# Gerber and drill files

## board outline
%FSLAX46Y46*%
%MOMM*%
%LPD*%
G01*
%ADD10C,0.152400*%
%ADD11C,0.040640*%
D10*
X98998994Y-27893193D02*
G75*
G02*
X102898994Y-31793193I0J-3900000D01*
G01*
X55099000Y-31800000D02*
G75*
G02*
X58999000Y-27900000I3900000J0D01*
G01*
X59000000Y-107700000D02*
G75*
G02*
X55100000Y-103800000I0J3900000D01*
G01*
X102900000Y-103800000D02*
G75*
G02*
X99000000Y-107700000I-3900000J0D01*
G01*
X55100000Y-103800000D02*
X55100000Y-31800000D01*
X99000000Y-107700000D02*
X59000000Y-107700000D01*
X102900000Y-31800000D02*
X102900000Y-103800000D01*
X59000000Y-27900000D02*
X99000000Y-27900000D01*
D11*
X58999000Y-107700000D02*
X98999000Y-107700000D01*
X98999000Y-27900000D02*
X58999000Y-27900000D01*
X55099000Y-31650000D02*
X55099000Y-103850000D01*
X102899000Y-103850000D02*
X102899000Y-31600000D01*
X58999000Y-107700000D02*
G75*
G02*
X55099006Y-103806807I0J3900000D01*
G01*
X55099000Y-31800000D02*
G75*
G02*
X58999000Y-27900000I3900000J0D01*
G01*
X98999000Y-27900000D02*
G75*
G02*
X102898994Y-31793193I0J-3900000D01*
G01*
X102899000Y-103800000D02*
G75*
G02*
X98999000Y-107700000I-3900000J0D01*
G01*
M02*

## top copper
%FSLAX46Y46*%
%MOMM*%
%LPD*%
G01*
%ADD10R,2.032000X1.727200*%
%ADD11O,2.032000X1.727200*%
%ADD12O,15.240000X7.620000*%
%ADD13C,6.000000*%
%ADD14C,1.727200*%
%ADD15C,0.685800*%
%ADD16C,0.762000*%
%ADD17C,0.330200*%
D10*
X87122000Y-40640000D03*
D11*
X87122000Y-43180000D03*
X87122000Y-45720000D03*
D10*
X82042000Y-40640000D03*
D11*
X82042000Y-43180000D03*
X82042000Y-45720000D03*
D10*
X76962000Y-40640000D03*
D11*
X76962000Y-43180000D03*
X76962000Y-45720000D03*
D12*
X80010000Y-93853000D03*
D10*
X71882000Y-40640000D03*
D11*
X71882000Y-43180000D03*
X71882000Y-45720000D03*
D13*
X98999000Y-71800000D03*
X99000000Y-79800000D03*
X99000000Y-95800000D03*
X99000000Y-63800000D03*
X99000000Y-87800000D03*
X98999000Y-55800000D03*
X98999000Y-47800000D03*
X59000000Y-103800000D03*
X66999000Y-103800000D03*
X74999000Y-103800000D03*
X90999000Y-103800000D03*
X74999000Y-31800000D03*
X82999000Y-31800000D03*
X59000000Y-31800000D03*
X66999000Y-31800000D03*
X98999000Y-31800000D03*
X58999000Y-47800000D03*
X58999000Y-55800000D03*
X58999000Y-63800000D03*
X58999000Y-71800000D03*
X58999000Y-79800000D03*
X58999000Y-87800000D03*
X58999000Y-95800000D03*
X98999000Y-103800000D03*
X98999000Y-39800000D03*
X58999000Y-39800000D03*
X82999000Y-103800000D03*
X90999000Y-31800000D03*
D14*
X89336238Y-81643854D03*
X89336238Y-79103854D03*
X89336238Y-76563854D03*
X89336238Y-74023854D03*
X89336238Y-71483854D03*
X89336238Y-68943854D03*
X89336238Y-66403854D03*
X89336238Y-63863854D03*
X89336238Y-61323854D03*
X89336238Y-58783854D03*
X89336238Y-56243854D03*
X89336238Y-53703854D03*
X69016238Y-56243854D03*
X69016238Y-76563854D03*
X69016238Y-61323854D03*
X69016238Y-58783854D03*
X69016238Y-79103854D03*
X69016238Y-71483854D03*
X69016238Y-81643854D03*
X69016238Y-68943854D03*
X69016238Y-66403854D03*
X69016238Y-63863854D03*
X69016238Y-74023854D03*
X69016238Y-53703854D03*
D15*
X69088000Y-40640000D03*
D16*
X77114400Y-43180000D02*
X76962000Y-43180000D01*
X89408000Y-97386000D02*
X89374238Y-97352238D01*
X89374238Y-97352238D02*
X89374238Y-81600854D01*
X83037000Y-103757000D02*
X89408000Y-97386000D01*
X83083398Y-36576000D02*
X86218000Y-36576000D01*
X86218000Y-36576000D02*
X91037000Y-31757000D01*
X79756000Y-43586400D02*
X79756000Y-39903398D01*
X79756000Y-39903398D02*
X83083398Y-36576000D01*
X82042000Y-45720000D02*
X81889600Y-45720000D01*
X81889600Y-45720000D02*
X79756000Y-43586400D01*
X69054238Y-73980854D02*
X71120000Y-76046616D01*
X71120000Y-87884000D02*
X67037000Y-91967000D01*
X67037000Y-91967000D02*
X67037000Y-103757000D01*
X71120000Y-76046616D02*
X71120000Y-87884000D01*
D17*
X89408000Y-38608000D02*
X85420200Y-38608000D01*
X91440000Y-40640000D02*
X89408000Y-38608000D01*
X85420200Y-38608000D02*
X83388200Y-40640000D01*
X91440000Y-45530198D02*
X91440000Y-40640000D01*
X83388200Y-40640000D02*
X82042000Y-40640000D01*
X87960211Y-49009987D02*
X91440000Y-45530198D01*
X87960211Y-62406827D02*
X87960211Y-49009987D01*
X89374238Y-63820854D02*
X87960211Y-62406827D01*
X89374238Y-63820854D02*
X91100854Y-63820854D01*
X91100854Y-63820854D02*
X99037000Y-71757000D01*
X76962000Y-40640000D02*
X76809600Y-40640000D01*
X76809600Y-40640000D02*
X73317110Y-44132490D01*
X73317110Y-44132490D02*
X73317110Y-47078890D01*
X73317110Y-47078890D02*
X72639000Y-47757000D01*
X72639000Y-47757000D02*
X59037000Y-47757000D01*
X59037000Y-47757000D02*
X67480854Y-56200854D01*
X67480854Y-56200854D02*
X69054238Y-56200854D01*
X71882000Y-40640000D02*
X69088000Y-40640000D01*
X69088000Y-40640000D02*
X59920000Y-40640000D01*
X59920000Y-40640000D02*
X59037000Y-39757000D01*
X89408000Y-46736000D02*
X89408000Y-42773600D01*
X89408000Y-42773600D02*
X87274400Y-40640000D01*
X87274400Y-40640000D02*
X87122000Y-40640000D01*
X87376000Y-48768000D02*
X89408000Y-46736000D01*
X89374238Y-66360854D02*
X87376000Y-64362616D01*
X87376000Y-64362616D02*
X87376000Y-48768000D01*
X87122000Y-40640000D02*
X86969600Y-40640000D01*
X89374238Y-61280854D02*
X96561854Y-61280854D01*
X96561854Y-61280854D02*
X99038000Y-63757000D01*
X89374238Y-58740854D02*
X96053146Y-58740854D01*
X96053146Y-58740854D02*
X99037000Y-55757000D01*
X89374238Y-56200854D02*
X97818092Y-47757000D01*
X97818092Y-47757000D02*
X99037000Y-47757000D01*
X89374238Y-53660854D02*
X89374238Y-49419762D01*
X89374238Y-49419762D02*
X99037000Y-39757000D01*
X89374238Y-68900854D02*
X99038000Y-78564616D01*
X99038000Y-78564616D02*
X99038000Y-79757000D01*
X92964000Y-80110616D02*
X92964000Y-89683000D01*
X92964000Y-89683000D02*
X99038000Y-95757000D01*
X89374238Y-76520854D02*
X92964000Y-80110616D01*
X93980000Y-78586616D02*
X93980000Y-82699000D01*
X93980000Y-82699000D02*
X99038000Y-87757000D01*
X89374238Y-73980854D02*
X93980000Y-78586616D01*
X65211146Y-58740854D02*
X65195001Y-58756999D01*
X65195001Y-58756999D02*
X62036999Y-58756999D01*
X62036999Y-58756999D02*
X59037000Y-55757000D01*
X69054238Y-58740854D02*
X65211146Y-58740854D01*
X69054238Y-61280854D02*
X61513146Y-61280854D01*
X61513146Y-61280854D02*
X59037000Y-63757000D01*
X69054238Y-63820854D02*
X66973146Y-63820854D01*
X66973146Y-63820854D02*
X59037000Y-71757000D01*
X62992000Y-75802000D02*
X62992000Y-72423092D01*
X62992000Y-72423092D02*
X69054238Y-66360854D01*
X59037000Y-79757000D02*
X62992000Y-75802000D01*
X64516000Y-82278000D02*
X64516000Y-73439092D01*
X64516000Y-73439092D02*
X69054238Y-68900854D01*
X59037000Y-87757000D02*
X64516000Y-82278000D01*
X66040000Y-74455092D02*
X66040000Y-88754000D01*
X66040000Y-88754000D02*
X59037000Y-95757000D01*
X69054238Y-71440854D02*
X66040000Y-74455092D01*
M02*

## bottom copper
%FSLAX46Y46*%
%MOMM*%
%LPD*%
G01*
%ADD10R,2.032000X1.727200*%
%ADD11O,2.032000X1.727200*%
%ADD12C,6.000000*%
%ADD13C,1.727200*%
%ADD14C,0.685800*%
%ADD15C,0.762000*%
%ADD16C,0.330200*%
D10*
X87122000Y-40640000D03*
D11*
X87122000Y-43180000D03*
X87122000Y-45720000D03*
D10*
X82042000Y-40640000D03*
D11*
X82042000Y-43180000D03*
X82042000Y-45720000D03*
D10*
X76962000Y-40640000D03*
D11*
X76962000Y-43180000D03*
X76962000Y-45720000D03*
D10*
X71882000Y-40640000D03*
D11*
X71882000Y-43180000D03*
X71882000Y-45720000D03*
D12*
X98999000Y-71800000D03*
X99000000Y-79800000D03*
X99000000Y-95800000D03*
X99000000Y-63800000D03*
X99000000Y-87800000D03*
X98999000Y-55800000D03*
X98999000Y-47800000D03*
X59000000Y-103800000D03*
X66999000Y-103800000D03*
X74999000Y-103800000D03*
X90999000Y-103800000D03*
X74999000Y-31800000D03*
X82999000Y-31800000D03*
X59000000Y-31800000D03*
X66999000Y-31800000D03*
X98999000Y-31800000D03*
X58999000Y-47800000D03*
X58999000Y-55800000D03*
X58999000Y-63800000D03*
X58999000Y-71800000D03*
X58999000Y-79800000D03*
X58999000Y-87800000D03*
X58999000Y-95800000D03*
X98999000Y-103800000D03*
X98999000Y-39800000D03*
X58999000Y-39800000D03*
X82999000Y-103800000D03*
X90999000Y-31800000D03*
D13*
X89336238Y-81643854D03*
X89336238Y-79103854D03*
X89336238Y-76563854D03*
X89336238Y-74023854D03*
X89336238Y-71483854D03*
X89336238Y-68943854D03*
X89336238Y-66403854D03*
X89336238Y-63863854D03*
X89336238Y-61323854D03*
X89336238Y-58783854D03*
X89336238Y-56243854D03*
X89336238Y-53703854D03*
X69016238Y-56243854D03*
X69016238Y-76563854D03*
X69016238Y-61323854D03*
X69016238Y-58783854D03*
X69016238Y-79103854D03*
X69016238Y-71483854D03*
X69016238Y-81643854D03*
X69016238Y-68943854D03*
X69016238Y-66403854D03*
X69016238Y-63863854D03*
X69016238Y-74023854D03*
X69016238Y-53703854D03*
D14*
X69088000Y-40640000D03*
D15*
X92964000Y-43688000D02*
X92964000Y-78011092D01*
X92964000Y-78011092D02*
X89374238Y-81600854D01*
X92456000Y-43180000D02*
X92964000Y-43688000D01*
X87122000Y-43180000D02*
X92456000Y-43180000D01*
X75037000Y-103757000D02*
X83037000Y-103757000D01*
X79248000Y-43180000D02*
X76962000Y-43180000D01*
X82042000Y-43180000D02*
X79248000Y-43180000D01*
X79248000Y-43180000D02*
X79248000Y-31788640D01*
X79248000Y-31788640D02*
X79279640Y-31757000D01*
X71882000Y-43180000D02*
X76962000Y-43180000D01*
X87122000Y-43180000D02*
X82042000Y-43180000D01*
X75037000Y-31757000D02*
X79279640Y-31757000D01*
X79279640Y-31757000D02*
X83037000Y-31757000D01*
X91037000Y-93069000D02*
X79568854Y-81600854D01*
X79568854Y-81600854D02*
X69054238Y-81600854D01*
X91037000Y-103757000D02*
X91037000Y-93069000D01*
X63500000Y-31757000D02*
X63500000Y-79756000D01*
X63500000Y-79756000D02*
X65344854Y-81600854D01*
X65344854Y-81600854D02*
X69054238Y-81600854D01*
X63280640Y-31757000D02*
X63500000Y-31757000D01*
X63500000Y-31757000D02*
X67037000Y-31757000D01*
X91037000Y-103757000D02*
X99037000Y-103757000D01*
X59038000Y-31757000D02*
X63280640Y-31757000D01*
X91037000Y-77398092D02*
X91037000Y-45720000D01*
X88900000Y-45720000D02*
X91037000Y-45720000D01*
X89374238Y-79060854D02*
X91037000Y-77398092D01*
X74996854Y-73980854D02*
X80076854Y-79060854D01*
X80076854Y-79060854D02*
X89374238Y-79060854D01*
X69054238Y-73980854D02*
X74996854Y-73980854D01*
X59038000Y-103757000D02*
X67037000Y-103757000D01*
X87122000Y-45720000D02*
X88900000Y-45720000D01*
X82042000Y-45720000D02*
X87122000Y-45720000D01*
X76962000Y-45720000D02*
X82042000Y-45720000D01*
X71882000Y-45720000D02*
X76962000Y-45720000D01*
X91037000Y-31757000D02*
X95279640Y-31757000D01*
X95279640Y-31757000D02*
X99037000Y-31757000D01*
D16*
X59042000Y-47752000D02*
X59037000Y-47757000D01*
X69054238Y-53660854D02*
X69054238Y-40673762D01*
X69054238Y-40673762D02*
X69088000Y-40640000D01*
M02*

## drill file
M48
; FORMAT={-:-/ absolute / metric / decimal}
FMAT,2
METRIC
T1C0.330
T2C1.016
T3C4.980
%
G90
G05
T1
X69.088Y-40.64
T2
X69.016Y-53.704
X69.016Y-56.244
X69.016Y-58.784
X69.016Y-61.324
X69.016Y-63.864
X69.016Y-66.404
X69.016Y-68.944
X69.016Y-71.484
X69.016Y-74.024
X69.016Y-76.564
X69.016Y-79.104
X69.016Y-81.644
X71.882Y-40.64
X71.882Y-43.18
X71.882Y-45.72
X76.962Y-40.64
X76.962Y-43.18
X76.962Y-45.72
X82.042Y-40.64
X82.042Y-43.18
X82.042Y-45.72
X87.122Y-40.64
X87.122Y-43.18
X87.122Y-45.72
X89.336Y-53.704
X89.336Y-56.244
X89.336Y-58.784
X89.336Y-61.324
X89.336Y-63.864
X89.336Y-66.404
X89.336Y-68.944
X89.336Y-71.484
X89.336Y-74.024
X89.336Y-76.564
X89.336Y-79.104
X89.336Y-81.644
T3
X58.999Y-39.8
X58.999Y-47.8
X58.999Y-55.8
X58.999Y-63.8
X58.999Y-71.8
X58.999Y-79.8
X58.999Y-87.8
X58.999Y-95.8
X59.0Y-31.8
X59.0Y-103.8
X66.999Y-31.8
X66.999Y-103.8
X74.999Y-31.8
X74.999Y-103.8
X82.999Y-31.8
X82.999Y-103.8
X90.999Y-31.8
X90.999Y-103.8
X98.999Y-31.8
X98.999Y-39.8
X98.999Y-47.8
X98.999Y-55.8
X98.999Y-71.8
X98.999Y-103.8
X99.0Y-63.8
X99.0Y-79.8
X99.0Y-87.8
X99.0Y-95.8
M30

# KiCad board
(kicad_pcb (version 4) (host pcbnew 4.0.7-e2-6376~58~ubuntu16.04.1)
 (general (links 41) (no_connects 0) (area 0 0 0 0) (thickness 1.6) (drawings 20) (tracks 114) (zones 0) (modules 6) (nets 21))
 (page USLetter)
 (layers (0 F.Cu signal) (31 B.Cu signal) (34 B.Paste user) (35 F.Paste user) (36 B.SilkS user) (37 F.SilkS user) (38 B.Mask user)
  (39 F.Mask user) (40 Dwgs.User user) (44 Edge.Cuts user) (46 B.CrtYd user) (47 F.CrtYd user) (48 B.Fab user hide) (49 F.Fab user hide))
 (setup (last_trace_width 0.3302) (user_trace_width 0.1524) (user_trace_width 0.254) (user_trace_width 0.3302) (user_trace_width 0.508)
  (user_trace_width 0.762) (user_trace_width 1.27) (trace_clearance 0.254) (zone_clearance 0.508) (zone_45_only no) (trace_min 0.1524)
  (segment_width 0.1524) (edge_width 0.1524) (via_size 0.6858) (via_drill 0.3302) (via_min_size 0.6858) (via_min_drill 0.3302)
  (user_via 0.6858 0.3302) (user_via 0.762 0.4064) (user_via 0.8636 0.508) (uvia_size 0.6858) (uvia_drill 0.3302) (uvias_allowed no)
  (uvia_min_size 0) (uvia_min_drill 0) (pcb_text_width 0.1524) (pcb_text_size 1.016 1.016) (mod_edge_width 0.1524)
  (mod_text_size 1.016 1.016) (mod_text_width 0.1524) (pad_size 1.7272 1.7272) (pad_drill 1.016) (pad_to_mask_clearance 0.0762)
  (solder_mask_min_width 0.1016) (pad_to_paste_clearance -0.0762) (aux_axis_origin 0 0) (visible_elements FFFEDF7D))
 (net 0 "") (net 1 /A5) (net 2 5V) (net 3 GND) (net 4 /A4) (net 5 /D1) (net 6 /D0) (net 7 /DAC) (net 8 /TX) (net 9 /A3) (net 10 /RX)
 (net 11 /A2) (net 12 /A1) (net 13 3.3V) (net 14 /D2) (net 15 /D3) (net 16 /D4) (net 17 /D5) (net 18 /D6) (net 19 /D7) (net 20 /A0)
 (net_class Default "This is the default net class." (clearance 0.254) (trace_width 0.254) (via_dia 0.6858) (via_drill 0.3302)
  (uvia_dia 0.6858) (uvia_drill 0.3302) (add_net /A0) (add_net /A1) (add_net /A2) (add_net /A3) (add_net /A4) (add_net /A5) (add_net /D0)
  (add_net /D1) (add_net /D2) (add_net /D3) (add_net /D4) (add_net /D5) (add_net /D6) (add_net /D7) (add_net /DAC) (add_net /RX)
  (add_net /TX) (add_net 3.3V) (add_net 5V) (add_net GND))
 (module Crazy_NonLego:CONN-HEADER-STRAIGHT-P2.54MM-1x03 (layer F.Cu) (at 87.122 40.64)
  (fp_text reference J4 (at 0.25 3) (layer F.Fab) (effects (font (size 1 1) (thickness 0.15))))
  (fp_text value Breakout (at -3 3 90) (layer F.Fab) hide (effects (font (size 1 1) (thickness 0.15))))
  (pad A5 thru_hole rect (at 0 0) (size 2.032 1.7272) (drill 1.016) (layers *.Cu *.Mask F.SilkS) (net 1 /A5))
  (pad VIN thru_hole oval (at 0 2.54) (size 2.032 1.7272) (drill 1.016) (layers *.Cu *.Mask F.SilkS) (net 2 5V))
  (pad GND thru_hole oval (at 0 5.08) (size 2.032 1.7272) (drill 1.016) (layers *.Cu *.Mask F.SilkS) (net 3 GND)))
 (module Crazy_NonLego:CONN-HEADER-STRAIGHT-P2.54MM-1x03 (layer F.Cu) (at 82.042 40.64)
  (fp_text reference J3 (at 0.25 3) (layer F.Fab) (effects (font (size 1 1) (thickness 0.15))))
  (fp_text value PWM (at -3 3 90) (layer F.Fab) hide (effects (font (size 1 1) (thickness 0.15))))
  (pad A4 thru_hole rect (at 0 0) (size 2.032 1.7272) (drill 1.016) (layers *.Cu *.Mask F.SilkS) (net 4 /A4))
  (pad VIN thru_hole oval (at 0 2.54) (size 2.032 1.7272) (drill 1.016) (layers *.Cu *.Mask F.SilkS) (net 2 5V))
  (pad GND thru_hole oval (at 0 5.08) (size 2.032 1.7272) (drill 1.016) (layers *.Cu *.Mask F.SilkS) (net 3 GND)))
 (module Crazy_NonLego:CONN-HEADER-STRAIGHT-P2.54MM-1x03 (layer F.Cu) (at 76.962 40.64)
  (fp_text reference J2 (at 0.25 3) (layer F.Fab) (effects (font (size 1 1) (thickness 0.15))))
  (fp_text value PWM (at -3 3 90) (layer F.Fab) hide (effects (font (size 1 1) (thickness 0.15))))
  (pad D1 thru_hole rect (at 0 0) (size 2.032 1.7272) (drill 1.016) (layers *.Cu *.Mask F.SilkS) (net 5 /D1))
  (pad VIN thru_hole oval (at 0 2.54) (size 2.032 1.7272) (drill 1.016) (layers *.Cu *.Mask F.SilkS) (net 2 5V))
  (pad GND thru_hole oval (at 0 5.08) (size 2.032 1.7272) (drill 1.016) (layers *.Cu *.Mask F.SilkS) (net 3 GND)))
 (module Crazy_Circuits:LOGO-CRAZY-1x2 (layer F.Cu) (at 80.01 97.79)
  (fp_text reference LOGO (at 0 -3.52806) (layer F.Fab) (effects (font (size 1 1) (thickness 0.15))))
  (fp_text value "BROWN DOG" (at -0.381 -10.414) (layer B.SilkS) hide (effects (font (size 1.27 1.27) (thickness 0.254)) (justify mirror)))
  (pad BG smd oval (at 0 -3.937) (size 15.24 7.62) (layers F.Cu)))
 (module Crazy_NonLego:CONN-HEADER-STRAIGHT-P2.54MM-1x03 (layer F.Cu) (at 71.882 40.64)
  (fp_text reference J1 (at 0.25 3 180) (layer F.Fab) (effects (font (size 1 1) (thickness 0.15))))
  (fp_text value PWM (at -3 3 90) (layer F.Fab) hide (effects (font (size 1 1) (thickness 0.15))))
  (pad D0 thru_hole rect (at 0 0) (size 2.032 1.7272) (drill 1.016) (layers *.Cu *.Mask F.SilkS) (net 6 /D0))
  (pad VIN thru_hole oval (at 0 2.54) (size 2.032 1.7272) (drill 1.016) (layers *.Cu *.Mask F.SilkS) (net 2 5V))
  (pad GND thru_hole oval (at 0 5.08) (size 2.032 1.7272) (drill 1.016) (layers *.Cu *.Mask F.SilkS) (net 3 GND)))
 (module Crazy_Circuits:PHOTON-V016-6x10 (layer F.Cu) (at 58.999 103.8)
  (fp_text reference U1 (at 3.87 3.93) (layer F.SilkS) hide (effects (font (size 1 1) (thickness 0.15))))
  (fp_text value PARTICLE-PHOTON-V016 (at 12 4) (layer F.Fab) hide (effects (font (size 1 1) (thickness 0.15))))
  (fp_line (start 0 3.9) (end 40 3.9) (layer Edge.Cuts) (width 0.04064))
  (fp_line (start 40 -75.9) (end 0 -75.9) (layer Edge.Cuts) (width 0.04064))
  (fp_line (start -3.9 -72.15) (end -3.9 0.05) (layer Edge.Cuts) (width 0.04064))
  (fp_line (start 43.9 0.05) (end 43.9 -72.2) (layer Edge.Cuts) (width 0.04064))
  (fp_arc (start 0 0) (end 0 3.9) (angle 89.9) (layer Edge.Cuts) (width 0.04064))
  (fp_arc (start 0 -72) (end -3.9 -72) (angle 90) (layer Edge.Cuts) (width 0.04064))
  (fp_arc (start 40 -72) (end 40 -75.9) (angle 89.9) (layer Edge.Cuts) (width 0.04064))
  (fp_arc (start 40 0) (end 43.9 0) (angle 90) (layer Edge.Cuts) (width 0.04064))
  (pad A4 thru_hole circle (at 40 -32 90) (size 6 6) (drill 4.98) (layers *.Cu *.Mask) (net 4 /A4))
  (pad DAC thru_hole circle (at 40.001 -24 90) (size 6 6) (drill 4.98) (layers *.Cu *.Mask) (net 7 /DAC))
  (pad TX thru_hole circle (at 40.001 -8 90) (size 6 6) (drill 4.98) (layers *.Cu *.Mask) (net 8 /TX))
  (pad A3 thru_hole circle (at 40.001 -40 90) (size 6 6) (drill 4.98) (layers *.Cu *.Mask) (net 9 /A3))
  (pad RX thru_hole circle (at 40.001 -16 90) (size 6 6) (drill 4.98) (layers *.Cu *.Mask) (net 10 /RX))
  (pad A2 thru_hole circle (at 40 -48 90) (size 6 6) (drill 4.98) (layers *.Cu *.Mask) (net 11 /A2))
  (pad A1 thru_hole circle (at 40 -56 90) (size 6 6) (drill 4.98) (layers *.Cu *.Mask) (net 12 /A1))
  (pad GND thru_hole circle (at 0.001 0 90) (size 6 6) (drill 4.98) (layers *.Cu *.Mask) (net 3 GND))
  (pad GND thru_hole circle (at 8 0 90) (size 6 6) (drill 4.98) (layers *.Cu *.Mask) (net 3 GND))
  (pad 5V thru_hole circle (at 16 0 90) (size 6 6) (drill 4.98) (layers *.Cu *.Mask) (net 2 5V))
  (pad 3V thru_hole circle (at 32 0 90) (size 6 6) (drill 4.98) (layers *.Cu *.Mask) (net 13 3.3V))
  (pad 5V thru_hole circle (at 16 -72 90) (size 6 6) (drill 4.98) (layers *.Cu *.Mask) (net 2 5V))
  (pad 5V thru_hole circle (at 24 -72 90) (size 6 6) (drill 4.98) (layers *.Cu *.Mask) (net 2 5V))
  (pad 3V thru_hole circle (at 0.001 -72 90) (size 6 6) (drill 4.98) (layers *.Cu *.Mask) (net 13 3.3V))
  (pad 3V thru_hole circle (at 8 -72 90) (size 6 6) (drill 4.98) (layers *.Cu *.Mask) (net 13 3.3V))
  (pad GND thru_hole circle (at 40 -72 90) (size 6 6) (drill 4.98) (layers *.Cu *.Mask) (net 3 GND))
  (pad D1 thru_hole circle (at 0 -56 90) (size 6 6) (drill 4.98) (layers *.Cu *.Mask) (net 5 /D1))
  (pad D2 thru_hole circle (at 0 -48 90) (size 6 6) (drill 4.98) (layers *.Cu *.Mask) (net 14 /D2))
  (pad D3 thru_hole circle (at 0 -40 90) (size 6 6) (drill 4.98) (layers *.Cu *.Mask) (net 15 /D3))
  (pad D4 thru_hole circle (at 0 -32 90) (size 6 6) (drill 4.98) (layers *.Cu *.Mask) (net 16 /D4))
  (pad D5 thru_hole circle (at 0 -24 90) (size 6 6) (drill 4.98) (layers *.Cu *.Mask) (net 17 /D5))
  (pad D6 thru_hole circle (at 0 -16 90) (size 6 6) (drill 4.98) (layers *.Cu *.Mask) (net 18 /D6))
  (pad D7 thru_hole circle (at 0 -8 90) (size 6 6) (drill 4.98) (layers *.Cu *.Mask) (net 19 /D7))
  (pad 3V thru_hole circle (at 40 0 90) (size 6 6) (drill 4.98) (layers *.Cu *.Mask) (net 13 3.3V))
  (pad A0 thru_hole circle (at 40 -64 90) (size 6 6) (drill 4.98) (layers *.Cu *.Mask) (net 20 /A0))
  (pad D0 thru_hole circle (at 0 -64 90) (size 6 6) (drill 4.98) (layers *.Cu *.Mask) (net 6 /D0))
  (pad 5V thru_hole circle (at 24 0 90) (size 6 6) (drill 4.98) (layers *.Cu *.Mask) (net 2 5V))
  (pad GND thru_hole circle (at 32 -72 90) (size 6 6) (drill 4.98) (layers *.Cu *.Mask) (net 3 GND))
  (pad VIN thru_hole circle (at 30.337238 -22.156146 180) (size 1.7272 1.7272) (drill 1.016) (layers *.Cu *.Mask F.SilkS) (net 2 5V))
  (pad GND thru_hole circle (at 30.337238 -24.696146 180) (size 1.7272 1.7272) (drill 1.016) (layers *.Cu *.Mask F.SilkS) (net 3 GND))
  (pad TX thru_hole circle (at 30.337238 -27.236146 180) (size 1.7272 1.7272) (drill 1.016) (layers *.Cu *.Mask F.SilkS) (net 8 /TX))
  (pad RX thru_hole circle (at 30.337238 -29.776146 180) (size 1.7272 1.7272) (drill 1.016) (layers *.Cu *.Mask F.SilkS) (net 10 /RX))
  (pad WKP thru_hole circle (at 30.337238 -32.316146 180) (size 1.7272 1.7272) (drill 1.016) (layers *.Cu *.Mask F.SilkS))
  (pad DAC thru_hole circle (at 30.337238 -34.856146 180) (size 1.7272 1.7272) (drill 1.016) (layers *.Cu *.Mask F.SilkS) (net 7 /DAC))
  (pad A5 thru_hole circle (at 30.337238 -37.396146 180) (size 1.7272 1.7272) (drill 1.016) (layers *.Cu *.Mask F.SilkS) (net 1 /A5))
  (pad A4 thru_hole circle (at 30.337238 -39.936146 180) (size 1.7272 1.7272) (drill 1.016) (layers *.Cu *.Mask F.SilkS) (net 4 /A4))
  (pad A3 thru_hole circle (at 30.337238 -42.476146 180) (size 1.7272 1.7272) (drill 1.016) (layers *.Cu *.Mask F.SilkS) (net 9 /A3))
  (pad A2 thru_hole circle (at 30.337238 -45.016146 180) (size 1.7272 1.7272) (drill 1.016) (layers *.Cu *.Mask F.SilkS) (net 11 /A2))
  (pad A1 thru_hole circle (at 30.337238 -47.556146 180) (size 1.7272 1.7272) (drill 1.016) (layers *.Cu *.Mask F.SilkS) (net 12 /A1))
  (pad A0 thru_hole circle (at 30.337238 -50.096146 180) (size 1.7272 1.7272) (drill 1.016) (layers *.Cu *.Mask F.SilkS) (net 20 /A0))
  (pad D1 thru_hole circle (at 10.017238 -47.556146 180) (size 1.7272 1.7272) (drill 1.016) (layers *.Cu *.Mask F.SilkS) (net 5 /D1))
  (pad VBAT thru_hole circle (at 10.017238 -27.236146 180) (size 1.7272 1.7272) (drill 1.016) (layers *.Cu *.Mask F.SilkS))
  (pad D3 thru_hole circle (at 10.017238 -42.476146 180) (size 1.7272 1.7272) (drill 1.016) (layers *.Cu *.Mask F.SilkS) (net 15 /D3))
  (pad D2 thru_hole circle (at 10.017238 -45.016146 180) (size 1.7272 1.7272) (drill 1.016) (layers *.Cu *.Mask F.SilkS) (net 14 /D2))
  (pad RST thru_hole circle (at 10.017238 -24.696146 180) (size 1.7272 1.7272) (drill 1.016) (layers *.Cu *.Mask F.SilkS))
  (pad D7 thru_hole circle (at 10.017238 -32.316146 180) (size 1.7272 1.7272) (drill 1.016) (layers *.Cu *.Mask F.SilkS) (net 19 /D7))
  (pad 3V thru_hole circle (at 10.017238 -22.156146 180) (size 1.7272 1.7272) (drill 1.016) (layers *.Cu *.Mask F.SilkS) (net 13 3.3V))
  (pad D6 thru_hole circle (at 10.017238 -34.856146 180) (size 1.7272 1.7272) (drill 1.016) (layers *.Cu *.Mask F.SilkS) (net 18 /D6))
  (pad D5 thru_hole circle (at 10.017238 -37.396146 180) (size 1.7272 1.7272) (drill 1.016) (layers *.Cu *.Mask F.SilkS) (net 17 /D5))
  (pad D4 thru_hole circle (at 10.017238 -39.936146 180) (size 1.7272 1.7272) (drill 1.016) (layers *.Cu *.Mask F.SilkS) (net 16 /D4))
  (pad GND thru_hole circle (at 10.017238 -29.776146 180) (size 1.7272 1.7272) (drill 1.016) (layers *.Cu *.Mask F.SilkS) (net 3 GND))
  (pad D0 thru_hole circle (at 10.017238 -50.096146 180) (size 1.7272 1.7272) (drill 1.016) (layers *.Cu *.Mask F.SilkS) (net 6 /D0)))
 (gr_arc (start 98.998994 31.793193) (end 98.998994 27.893193) (angle 90) (layer Edge.Cuts) (width 0.1524))
 (gr_arc (start 58.999 31.8) (end 55.099 31.8) (angle 90) (layer Edge.Cuts) (width 0.1524))
 (gr_arc (start 59 103.8) (end 59 107.7) (angle 90) (layer Edge.Cuts) (width 0.1524))
 (gr_arc (start 99 103.8) (end 102.9 103.8) (angle 90) (layer Edge.Cuts) (width 0.1524))
 (gr_line (start 55.1 103.8) (end 55.1 31.8) (layer Edge.Cuts) (width 0.1524))
 (gr_line (start 99 107.7) (end 59 107.7) (layer Edge.Cuts) (width 0.1524))
 (gr_line (start 102.9 31.8) (end 102.9 103.8) (layer Edge.Cuts) (width 0.1524))
 (gr_line (start 59 27.9) (end 99 27.9) (layer Edge.Cuts) (width 0.1524))
 (segment (start 92.964 43.688) (end 92.964 78.011092) (width 0.762) (layer B.Cu) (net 2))
 (segment (start 92.964 78.011092) (end 89.374238 81.600854) (width 0.762) (layer B.Cu) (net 2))
 (segment (start 92.456 43.18) (end 92.964 43.688) (width 0.762) (layer B.Cu) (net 2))
 (segment (start 87.122 43.18) (end 92.456 43.18) (width 0.762) (layer B.Cu) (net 2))
 (segment (start 77.1144 43.18) (end 76.962 43.18) (width 0.762) (layer F.Cu) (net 2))
 (segment (start 89.408 97.386) (end 89.374238 97.352238) (width 0.762) (layer F.Cu) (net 2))
 (segment (start 89.374238 97.352238) (end 89.374238 81.600854) (width 0.762) (layer F.Cu) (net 2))
 (segment (start 83.037 103.757) (end 89.408 97.386) (width 0.762) (layer F.Cu) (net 2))
 (segment (start 75.037 103.757) (end 83.037 103.757) (width 0.762) (layer B.Cu) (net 2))
 (segment (start 79.248 43.18) (end 76.962 43.18) (width 0.762) (layer B.Cu) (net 2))
 (segment (start 82.042 43.18) (end 79.248 43.18) (width 0.762) (layer B.Cu) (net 2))
 (segment (start 79.248 43.18) (end 79.248 31.78864) (width 0.762) (layer B.Cu) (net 2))
 (segment (start 79.248 31.78864) (end 79.27964 31.757) (width 0.762) (layer B.Cu) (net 2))
 (segment (start 71.882 43.18) (end 76.962 43.18) (width 0.762) (layer B.Cu) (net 2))
 (segment (start 87.122 43.18) (end 82.042 43.18) (width 0.762) (layer B.Cu) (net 2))
 (segment (start 75.037 31.757) (end 79.27964 31.757) (width 0.762) (layer B.Cu) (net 2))
 (segment (start 79.27964 31.757) (end 83.037 31.757) (width 0.762) (layer B.Cu) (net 2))
 (segment (start 91.037 93.069) (end 79.568854 81.600854) (width 0.762) (layer B.Cu) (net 13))
 (segment (start 79.568854 81.600854) (end 69.054238 81.600854) (width 0.762) (layer B.Cu) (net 13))
 (segment (start 91.037 103.757) (end 91.037 93.069) (width 0.762) (layer B.Cu) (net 13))
 (segment (start 63.5 31.757) (end 63.5 79.756) (width 0.762) (layer B.Cu) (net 13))
 (segment (start 63.5 79.756) (end 65.344854 81.600854) (width 0.762) (layer B.Cu) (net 13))
 (segment (start 65.344854 81.600854) (end 69.054238 81.600854) (width 0.762) (layer B.Cu) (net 13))
 (segment (start 63.28064 31.757) (end 63.5 31.757) (width 0.762) (layer B.Cu) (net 13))
 (segment (start 63.5 31.757) (end 67.037 31.757) (width 0.762) (layer B.Cu) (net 13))
 (segment (start 91.037 103.757) (end 99.037 103.757) (width 0.762) (layer B.Cu) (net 13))
 (segment (start 59.038 31.757) (end 63.28064 31.757) (width 0.762) (layer B.Cu) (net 13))
 (segment (start 83.083398 36.576) (end 86.218 36.576) (width 0.762) (layer F.Cu) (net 3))
 (segment (start 86.218 36.576) (end 91.037 31.757) (width 0.762) (layer F.Cu) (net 3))
 (segment (start 79.756 43.5864) (end 79.756 39.903398) (width 0.762) (layer F.Cu) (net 3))
 (segment (start 79.756 39.903398) (end 83.083398 36.576) (width 0.762) (layer F.Cu) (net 3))
 (segment (start 82.042 45.72) (end 81.8896 45.72) (width 0.762) (layer F.Cu) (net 3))
 (segment (start 81.8896 45.72) (end 79.756 43.5864) (width 0.762) (layer F.Cu) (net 3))
 (segment (start 69.054238 73.980854) (end 71.12 76.046616) (width 0.762) (layer F.Cu) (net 3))
 (segment (start 91.037 77.398092) (end 91.037 45.72) (width 0.762) (layer B.Cu) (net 3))
 (segment (start 88.9 45.72) (end 91.037 45.72) (width 0.762) (layer B.Cu) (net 3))
 (segment (start 89.374238 79.060854) (end 91.037 77.398092) (width 0.762) (layer B.Cu) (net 3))
 (segment (start 71.12 87.884) (end 67.037 91.967) (width 0.762) (layer F.Cu) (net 3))
 (segment (start 67.037 91.967) (end 67.037 103.757) (width 0.762) (layer F.Cu) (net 3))
 (segment (start 71.12 76.046616) (end 71.12 87.884) (width 0.762) (layer F.Cu) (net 3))
 (segment (start 74.996854 73.980854) (end 80.076854 79.060854) (width 0.762) (layer B.Cu) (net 3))
 (segment (start 80.076854 79.060854) (end 89.374238 79.060854) (width 0.762) (layer B.Cu) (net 3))
 (segment (start 69.054238 73.980854) (end 74.996854 73.980854) (width 0.762) (layer B.Cu) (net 3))
 (segment (start 59.038 103.757) (end 67.037 103.757) (width 0.762) (layer B.Cu) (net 3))
 (segment (start 87.122 45.72) (end 88.9 45.72) (width 0.762) (layer B.Cu) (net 3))
 (segment (start 82.042 45.72) (end 87.122 45.72) (width 0.762) (layer B.Cu) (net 3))
 (segment (start 76.962 45.72) (end 82.042 45.72) (width 0.762) (layer B.Cu) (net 3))
 (segment (start 71.882 45.72) (end 76.962 45.72) (width 0.762) (layer B.Cu) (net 3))
 (segment (start 91.037 31.757) (end 95.27964 31.757) (width 0.762) (layer B.Cu) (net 3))
 (segment (start 95.27964 31.757) (end 99.037 31.757) (width 0.762) (layer B.Cu) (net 3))
 (segment (start 89.408 38.608) (end 85.4202 38.608) (width 0.3302) (layer F.Cu) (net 4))
 (segment (start 91.44 40.64) (end 89.408 38.608) (width 0.3302) (layer F.Cu) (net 4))
 (segment (start 85.4202 38.608) (end 83.3882 40.64) (width 0.3302) (layer F.Cu) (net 4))
 (segment (start 91.44 45.530198) (end 91.44 40.64) (width 0.3302) (layer F.Cu) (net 4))
 (segment (start 83.3882 40.64) (end 82.042 40.64) (width 0.3302) (layer F.Cu) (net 4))
 (segment (start 87.960211 49.009987) (end 91.44 45.530198) (width 0.3302) (layer F.Cu) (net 4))
 (segment (start 87.960211 62.406827) (end 87.960211 49.009987) (width 0.3302) (layer F.Cu) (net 4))
 (segment (start 89.374238 63.820854) (end 87.960211 62.406827) (width 0.3302) (layer F.Cu) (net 4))
 (segment (start 89.374238 63.820854) (end 91.100854 63.820854) (width 0.3302) (layer F.Cu) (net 4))
 (segment (start 91.100854 63.820854) (end 99.037 71.757) (width 0.3302) (layer F.Cu) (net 4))
 (segment (start 76.962 40.64) (end 76.8096 40.64) (width 0.3302) (layer F.Cu) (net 5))
 (segment (start 76.8096 40.64) (end 73.31711 44.13249) (width 0.3302) (layer F.Cu) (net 5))
 (segment (start 73.31711 44.13249) (end 73.31711 47.07889) (width 0.3302) (layer F.Cu) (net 5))
 (segment (start 73.31711 47.07889) (end 72.639 47.757) (width 0.3302) (layer F.Cu) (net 5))
 (segment (start 72.639 47.757) (end 59.037 47.757) (width 0.3302) (layer F.Cu) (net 5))
 (segment (start 59.042 47.752) (end 59.037 47.757) (width 0.3302) (layer B.Cu) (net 5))
 (segment (start 59.037 47.757) (end 67.480854 56.200854) (width 0.3302) (layer F.Cu) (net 5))
 (segment (start 67.480854 56.200854) (end 69.054238 56.200854) (width 0.3302) (layer F.Cu) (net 5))
 (segment (start 71.882 40.64) (end 69.088 40.64) (width 0.3302) (layer F.Cu) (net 6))
 (segment (start 69.088 40.64) (end 59.92 40.64) (width 0.3302) (layer F.Cu) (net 6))
 (segment (start 69.054238 53.660854) (end 69.054238 40.673762) (width 0.3302) (layer B.Cu) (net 6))
 (via (at 69.088 40.64) (size 0.6858) (drill 0.3302) (layers F.Cu B.Cu) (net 6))
 (segment (start 69.054238 40.673762) (end 69.088 40.64) (width 0.3302) (layer B.Cu) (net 6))
 (segment (start 59.92 40.64) (end 59.037 39.757) (width 0.3302) (layer F.Cu) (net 6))
 (segment (start 89.408 46.736) (end 89.408 42.7736) (width 0.3302) (layer F.Cu) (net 1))
 (segment (start 89.408 42.7736) (end 87.2744 40.64) (width 0.3302) (layer F.Cu) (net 1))
 (segment (start 87.2744 40.64) (end 87.122 40.64) (width 0.3302) (layer F.Cu) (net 1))
 (segment (start 87.376 48.768) (end 89.408 46.736) (width 0.3302) (layer F.Cu) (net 1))
 (segment (start 89.374238 66.360854) (end 87.376 64.362616) (width 0.3302) (layer F.Cu) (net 1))
 (segment (start 87.376 64.362616) (end 87.376 48.768) (width 0.3302) (layer F.Cu) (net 1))
 (segment (start 87.122 40.64) (end 86.9696 40.64) (width 0.3302) (layer F.Cu) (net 1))
 (segment (start 89.374238 61.280854) (end 96.561854 61.280854) (width 0.3302) (layer F.Cu) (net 9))
 (segment (start 96.561854 61.280854) (end 99.038 63.757) (width 0.3302) (layer F.Cu) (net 9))
 (segment (start 89.374238 58.740854) (end 96.053146 58.740854) (width 0.3302) (layer F.Cu) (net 11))
 (segment (start 96.053146 58.740854) (end 99.037 55.757) (width 0.3302) (layer F.Cu) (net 11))
 (segment (start 89.374238 56.200854) (end 97.818092 47.757) (width 0.3302) (layer F.Cu) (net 12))
 (segment (start 97.818092 47.757) (end 99.037 47.757) (width 0.3302) (layer F.Cu) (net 12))
 (segment (start 89.374238 53.660854) (end 89.374238 49.419762) (width 0.3302) (layer F.Cu) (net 20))
 (segment (start 89.374238 49.419762) (end 99.037 39.757) (width 0.3302) (layer F.Cu) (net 20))
 (segment (start 89.374238 68.900854) (end 99.038 78.564616) (width 0.3302) (layer F.Cu) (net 7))
 (segment (start 99.038 78.564616) (end 99.038 79.757) (width 0.3302) (layer F.Cu) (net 7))
 (segment (start 92.964 80.110616) (end 92.964 89.683) (width 0.3302) (layer F.Cu) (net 8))
 (segment (start 92.964 89.683) (end 99.038 95.757) (width 0.3302) (layer F.Cu) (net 8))
 (segment (start 89.374238 76.520854) (end 92.964 80.110616) (width 0.3302) (layer F.Cu) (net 8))
 (segment (start 93.98 78.586616) (end 93.98 82.699) (width 0.3302) (layer F.Cu) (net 10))
 (segment (start 93.98 82.699) (end 99.038 87.757) (width 0.3302) (layer F.Cu) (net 10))
 (segment (start 89.374238 73.980854) (end 93.98 78.586616) (width 0.3302) (layer F.Cu) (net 10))
 (segment (start 65.211146 58.740854) (end 65.195001 58.756999) (width 0.3302) (layer F.Cu) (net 14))
 (segment (start 65.195001 58.756999) (end 62.036999 58.756999) (width 0.3302) (layer F.Cu) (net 14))
 (segment (start 62.036999 58.756999) (end 59.037 55.757) (width 0.3302) (layer F.Cu) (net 14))
 (segment (start 69.054238 58.740854) (end 65.211146 58.740854) (width 0.3302) (layer F.Cu) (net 14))
 (segment (start 69.054238 61.280854) (end 61.513146 61.280854) (width 0.3302) (layer F.Cu) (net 15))
 (segment (start 61.513146 61.280854) (end 59.037 63.757) (width 0.3302) (layer F.Cu) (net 15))
 (segment (start 69.054238 63.820854) (end 66.973146 63.820854) (width 0.3302) (layer F.Cu) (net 16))
 (segment (start 66.973146 63.820854) (end 59.037 71.757) (width 0.3302) (layer F.Cu) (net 16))
 (segment (start 62.992 75.802) (end 62.992 72.423092) (width 0.3302) (layer F.Cu) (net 17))
 (segment (start 62.992 72.423092) (end 69.054238 66.360854) (width 0.3302) (layer F.Cu) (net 17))
 (segment (start 59.037 79.757) (end 62.992 75.802) (width 0.3302) (layer F.Cu) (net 17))
 (segment (start 64.516 82.278) (end 64.516 73.439092) (width 0.3302) (layer F.Cu) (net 18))
 (segment (start 64.516 73.439092) (end 69.054238 68.900854) (width 0.3302) (layer F.Cu) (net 18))
 (segment (start 59.037 87.757) (end 64.516 82.278) (width 0.3302) (layer F.Cu) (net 18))
 (segment (start 66.04 74.455092) (end 66.04 88.754) (width 0.3302) (layer F.Cu) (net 19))
 (segment (start 66.04 88.754) (end 59.037 95.757) (width 0.3302) (layer F.Cu) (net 19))
 (segment (start 69.054238 71.440854) (end 66.04 74.455092) (width 0.3302) (layer F.Cu) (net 19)))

